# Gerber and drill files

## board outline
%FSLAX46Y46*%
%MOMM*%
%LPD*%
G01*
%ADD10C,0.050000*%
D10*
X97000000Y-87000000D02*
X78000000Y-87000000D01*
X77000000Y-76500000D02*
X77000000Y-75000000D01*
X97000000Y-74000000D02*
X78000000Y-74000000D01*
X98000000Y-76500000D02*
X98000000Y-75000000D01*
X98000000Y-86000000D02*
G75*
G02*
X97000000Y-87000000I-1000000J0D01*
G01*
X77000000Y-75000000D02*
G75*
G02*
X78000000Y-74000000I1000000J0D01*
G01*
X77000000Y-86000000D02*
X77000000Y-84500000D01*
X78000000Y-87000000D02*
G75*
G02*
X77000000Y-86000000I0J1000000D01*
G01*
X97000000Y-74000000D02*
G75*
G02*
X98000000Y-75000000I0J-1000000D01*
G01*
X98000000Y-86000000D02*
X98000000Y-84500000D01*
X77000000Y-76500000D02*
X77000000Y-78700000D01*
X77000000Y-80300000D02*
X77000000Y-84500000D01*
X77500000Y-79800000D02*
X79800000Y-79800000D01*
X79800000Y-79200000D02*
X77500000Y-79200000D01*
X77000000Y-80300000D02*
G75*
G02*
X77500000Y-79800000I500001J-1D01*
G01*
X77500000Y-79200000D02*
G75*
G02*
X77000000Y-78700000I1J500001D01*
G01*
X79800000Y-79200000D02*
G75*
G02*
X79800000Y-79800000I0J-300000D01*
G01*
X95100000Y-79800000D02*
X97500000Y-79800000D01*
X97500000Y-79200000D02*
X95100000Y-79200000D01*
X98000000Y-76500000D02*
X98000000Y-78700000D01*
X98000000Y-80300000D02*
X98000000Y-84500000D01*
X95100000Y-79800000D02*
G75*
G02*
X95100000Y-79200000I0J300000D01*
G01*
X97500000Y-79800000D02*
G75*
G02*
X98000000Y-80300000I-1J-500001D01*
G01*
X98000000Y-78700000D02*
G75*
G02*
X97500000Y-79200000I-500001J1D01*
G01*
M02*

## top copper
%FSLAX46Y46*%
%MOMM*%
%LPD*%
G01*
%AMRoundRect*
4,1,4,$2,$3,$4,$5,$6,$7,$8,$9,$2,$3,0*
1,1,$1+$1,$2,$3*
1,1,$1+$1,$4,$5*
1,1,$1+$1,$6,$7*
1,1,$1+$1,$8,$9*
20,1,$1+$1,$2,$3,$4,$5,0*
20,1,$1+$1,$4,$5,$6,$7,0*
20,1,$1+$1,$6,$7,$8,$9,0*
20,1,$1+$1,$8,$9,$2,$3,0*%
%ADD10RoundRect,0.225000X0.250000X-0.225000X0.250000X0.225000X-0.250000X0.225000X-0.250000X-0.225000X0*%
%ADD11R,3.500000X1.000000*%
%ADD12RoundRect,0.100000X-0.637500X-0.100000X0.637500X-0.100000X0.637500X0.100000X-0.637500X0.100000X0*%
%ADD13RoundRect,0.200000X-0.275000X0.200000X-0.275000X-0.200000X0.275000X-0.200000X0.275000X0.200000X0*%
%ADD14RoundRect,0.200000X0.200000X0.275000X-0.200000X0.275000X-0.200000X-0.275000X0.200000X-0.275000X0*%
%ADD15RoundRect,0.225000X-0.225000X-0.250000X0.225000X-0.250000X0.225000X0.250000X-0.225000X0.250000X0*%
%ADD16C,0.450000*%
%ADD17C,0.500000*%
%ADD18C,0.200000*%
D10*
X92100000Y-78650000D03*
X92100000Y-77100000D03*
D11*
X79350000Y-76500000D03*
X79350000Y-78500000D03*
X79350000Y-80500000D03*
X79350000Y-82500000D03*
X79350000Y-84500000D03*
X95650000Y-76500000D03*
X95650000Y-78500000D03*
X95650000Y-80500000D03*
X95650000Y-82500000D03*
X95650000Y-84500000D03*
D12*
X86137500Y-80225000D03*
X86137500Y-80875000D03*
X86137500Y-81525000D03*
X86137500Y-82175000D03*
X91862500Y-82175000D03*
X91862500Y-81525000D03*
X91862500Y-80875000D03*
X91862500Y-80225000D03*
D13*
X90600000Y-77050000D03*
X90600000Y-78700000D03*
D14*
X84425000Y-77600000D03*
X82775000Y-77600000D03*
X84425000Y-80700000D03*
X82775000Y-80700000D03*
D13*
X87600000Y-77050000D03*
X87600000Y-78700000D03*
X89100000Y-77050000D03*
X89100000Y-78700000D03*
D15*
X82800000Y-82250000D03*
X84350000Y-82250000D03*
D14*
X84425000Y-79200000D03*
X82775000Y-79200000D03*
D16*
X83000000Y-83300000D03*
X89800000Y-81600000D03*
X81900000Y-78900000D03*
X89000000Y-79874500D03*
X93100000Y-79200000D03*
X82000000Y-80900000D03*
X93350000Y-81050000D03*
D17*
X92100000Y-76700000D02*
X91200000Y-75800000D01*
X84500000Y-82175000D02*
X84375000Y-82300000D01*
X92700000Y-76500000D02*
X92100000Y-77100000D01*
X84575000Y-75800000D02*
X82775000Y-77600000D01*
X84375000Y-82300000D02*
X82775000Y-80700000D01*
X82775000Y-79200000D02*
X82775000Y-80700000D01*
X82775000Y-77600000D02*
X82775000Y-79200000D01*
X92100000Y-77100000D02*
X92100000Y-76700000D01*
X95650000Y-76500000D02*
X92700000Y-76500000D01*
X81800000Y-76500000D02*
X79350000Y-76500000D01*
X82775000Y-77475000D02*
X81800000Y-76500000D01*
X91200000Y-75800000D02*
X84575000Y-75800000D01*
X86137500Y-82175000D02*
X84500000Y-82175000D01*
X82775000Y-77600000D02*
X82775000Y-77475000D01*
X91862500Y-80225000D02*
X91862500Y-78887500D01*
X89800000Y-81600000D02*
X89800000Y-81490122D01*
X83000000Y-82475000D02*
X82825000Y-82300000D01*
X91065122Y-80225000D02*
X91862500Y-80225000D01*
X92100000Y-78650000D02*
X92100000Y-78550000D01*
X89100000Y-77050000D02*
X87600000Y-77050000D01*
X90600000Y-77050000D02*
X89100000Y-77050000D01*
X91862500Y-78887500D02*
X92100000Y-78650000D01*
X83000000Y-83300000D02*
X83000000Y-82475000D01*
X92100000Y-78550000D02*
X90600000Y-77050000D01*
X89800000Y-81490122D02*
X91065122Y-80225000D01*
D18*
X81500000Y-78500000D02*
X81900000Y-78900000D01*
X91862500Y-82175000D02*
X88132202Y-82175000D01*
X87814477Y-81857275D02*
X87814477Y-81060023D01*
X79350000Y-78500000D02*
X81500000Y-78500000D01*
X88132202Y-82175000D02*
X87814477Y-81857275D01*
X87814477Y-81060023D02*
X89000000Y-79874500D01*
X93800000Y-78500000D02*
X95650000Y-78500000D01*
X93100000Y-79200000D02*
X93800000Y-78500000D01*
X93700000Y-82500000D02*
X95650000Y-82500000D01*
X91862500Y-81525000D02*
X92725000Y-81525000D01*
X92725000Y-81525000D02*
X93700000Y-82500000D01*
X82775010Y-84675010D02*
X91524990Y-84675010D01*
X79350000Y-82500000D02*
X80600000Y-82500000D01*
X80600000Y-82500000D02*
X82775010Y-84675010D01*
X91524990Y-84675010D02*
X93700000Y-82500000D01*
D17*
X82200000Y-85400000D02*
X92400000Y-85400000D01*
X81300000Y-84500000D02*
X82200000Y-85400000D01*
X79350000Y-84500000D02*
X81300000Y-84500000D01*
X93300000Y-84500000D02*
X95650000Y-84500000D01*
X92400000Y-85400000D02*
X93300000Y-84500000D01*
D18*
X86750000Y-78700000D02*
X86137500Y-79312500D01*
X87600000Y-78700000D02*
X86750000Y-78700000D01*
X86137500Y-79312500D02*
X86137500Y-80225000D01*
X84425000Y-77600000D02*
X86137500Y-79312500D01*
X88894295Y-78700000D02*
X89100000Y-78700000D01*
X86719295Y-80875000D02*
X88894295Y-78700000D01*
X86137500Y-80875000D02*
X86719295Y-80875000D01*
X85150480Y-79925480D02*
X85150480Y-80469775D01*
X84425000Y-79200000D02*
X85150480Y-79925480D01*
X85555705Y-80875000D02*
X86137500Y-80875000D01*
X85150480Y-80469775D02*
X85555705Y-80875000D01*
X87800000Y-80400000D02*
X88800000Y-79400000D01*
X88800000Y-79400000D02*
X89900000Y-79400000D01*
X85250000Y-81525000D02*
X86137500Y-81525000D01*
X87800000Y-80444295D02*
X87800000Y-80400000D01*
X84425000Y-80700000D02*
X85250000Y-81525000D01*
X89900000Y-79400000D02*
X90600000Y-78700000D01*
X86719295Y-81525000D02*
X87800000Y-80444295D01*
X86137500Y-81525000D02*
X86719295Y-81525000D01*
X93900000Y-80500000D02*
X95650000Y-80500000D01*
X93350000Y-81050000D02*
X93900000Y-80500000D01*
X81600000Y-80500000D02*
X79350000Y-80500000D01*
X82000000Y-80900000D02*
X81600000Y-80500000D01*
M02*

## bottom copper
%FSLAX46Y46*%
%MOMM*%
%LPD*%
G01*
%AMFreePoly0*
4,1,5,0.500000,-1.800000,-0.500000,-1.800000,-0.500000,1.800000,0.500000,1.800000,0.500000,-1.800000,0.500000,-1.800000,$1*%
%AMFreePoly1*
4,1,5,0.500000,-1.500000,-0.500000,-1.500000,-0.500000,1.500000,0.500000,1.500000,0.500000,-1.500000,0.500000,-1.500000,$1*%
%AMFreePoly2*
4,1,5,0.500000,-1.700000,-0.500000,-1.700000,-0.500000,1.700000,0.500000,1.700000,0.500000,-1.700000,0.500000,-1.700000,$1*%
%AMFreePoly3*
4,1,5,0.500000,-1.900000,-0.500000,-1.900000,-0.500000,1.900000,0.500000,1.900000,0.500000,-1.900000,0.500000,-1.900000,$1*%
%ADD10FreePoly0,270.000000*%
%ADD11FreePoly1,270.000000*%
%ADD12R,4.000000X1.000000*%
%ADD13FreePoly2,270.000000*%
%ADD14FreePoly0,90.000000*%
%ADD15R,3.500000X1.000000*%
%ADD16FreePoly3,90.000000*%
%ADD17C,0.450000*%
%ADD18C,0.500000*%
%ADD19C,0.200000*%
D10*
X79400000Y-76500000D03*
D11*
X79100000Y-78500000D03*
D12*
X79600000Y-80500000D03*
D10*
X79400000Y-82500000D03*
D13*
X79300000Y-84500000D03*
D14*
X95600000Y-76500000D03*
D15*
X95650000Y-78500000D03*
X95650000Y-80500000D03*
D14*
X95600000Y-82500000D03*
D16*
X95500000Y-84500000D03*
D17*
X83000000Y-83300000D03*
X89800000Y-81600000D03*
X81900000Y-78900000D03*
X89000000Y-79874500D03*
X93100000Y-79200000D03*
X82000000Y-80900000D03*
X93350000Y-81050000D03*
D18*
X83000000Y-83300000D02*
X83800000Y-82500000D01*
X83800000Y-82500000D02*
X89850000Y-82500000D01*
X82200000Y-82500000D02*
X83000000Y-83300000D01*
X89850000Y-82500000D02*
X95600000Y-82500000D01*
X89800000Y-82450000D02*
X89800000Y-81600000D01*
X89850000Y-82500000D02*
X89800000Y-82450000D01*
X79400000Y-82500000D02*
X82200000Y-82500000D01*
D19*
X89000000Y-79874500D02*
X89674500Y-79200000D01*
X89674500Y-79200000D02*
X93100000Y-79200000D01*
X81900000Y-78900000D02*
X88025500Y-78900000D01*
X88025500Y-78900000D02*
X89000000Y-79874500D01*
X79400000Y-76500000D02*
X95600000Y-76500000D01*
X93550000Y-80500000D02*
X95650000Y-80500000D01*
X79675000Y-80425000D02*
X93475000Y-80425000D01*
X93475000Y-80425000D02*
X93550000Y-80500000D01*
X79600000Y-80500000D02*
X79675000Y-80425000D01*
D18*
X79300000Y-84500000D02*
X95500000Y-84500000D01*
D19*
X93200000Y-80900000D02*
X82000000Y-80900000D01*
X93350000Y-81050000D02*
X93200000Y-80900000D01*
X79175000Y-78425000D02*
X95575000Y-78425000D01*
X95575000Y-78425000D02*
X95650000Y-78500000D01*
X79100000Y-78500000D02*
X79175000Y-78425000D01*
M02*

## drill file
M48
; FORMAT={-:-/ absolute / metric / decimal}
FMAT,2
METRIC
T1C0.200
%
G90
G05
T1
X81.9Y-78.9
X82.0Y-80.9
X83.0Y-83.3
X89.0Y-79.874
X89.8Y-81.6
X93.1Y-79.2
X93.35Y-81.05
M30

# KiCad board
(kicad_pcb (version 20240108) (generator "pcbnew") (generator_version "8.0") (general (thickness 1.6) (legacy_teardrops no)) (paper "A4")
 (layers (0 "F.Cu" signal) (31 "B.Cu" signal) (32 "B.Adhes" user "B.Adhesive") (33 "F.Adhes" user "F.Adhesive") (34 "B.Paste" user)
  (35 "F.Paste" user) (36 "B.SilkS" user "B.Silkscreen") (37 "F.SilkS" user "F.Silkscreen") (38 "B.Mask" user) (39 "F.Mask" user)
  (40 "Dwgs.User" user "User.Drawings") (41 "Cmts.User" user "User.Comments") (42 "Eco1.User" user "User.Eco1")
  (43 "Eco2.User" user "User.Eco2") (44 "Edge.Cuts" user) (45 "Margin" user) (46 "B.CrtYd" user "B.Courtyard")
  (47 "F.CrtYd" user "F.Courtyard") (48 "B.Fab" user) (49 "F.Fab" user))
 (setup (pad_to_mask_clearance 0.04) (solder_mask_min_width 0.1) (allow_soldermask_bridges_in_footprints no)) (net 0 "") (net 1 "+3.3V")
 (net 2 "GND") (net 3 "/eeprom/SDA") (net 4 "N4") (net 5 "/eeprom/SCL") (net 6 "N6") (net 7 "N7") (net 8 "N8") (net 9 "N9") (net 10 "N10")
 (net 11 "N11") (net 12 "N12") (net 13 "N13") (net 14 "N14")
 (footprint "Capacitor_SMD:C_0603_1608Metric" (layer "F.Cu") (at 92.1 77.875 90)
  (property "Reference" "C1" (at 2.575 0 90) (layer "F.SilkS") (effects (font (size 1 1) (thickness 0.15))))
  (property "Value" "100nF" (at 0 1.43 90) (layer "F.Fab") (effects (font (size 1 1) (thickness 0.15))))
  (pad "1" smd roundrect (at -0.775 0 90) (size 0.9 0.95) (layers "F.Cu" "F.Paste" "F.Mask") (roundrect_rratio 0.25) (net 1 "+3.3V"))
  (pad "2" smd roundrect (at 0.775 0 90) (size 0.9 0.95) (layers "F.Cu" "F.Paste" "F.Mask") (roundrect_rratio 0.25) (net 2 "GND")))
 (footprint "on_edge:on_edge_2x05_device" (layer "F.Cu") (at 77 80.5 -90)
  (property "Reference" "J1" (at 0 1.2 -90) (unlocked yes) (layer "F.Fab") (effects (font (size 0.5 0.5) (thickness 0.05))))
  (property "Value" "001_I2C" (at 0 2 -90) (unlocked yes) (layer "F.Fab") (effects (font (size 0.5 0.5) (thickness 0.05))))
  (fp_line (start -4 0) (end -1.8 0) (stroke (width 0.05) (type solid)) (layer "Edge.Cuts"))
  (fp_line (start -0.2 0) (end 4 0) (stroke (width 0.05) (type solid)) (layer "Edge.Cuts"))
  (fp_line (start -0.7 -0.5) (end -0.7 -2.8) (stroke (width 0.05) (type solid)) (layer "Edge.Cuts"))
  (fp_line (start -1.3 -2.8) (end -1.3 -0.5) (stroke (width 0.05) (type solid)) (layer "Edge.Cuts"))
  (fp_arc (start -0.2 0) (mid -0.553553 -0.146447) (end -0.7 -0.5) (stroke (width 0.05) (type solid)) (layer "Edge.Cuts"))
  (fp_arc (start -1.3 -0.5) (mid -1.446447 -0.146447) (end -1.8 0) (stroke (width 0.05) (type solid)) (layer "Edge.Cuts"))
  (fp_arc (start -1.3 -2.8) (mid -1 -3.1) (end -0.7 -2.8) (stroke (width 0.05) (type solid)) (layer "Edge.Cuts"))
  (pad "1" smd rect (at -4 -2.35 90) (size 1 3.5) (layers "F.Cu" "F.Mask") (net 2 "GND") (zone_connect 0))
  (pad "2" smd rect (at -2 -2.35 270) (size 1 3.5) (layers "F.Cu" "F.Mask") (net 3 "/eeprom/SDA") (zone_connect 0))
  (pad "3" smd rect (at 0 -2.35 270) (size 1 3.5) (layers "F.Cu" "F.Mask") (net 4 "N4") (zone_connect 0))
  (pad "4" smd rect (at 2 -2.35 90) (size 1 3.5) (layers "F.Cu" "F.Mask") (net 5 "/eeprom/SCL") (zone_connect 0))
  (pad "5" smd rect (at 4 -2.35 90) (size 1 3.5) (layers "F.Cu" "F.Mask") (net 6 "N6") (zone_connect 0))
  (pad "6" smd custom (at -4 -2.4 270) (size 1 3.6) (layers "B.Cu" "B.Mask") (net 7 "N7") (zone_connect 0)
   (options (clearance outline) (anchor rect)) (primitives))
  (pad "7" smd custom (at -2 -2.1 270) (size 1 3) (layers "B.Cu" "B.Mask") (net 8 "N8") (zone_connect 0)
   (options (clearance outline) (anchor rect)) (primitives))
  (pad "8" smd rect (at 0 -2.6 270) (size 1 4) (layers "B.Cu" "B.Mask") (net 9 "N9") (zone_connect 0))
  (pad "9" smd custom (at 2 -2.4 270) (size 1 3.6) (layers "B.Cu" "B.Mask") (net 1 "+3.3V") (zone_connect 0)
   (options (clearance outline) (anchor rect)) (primitives))
  (pad "10" smd custom (at 4 -2.3 270) (size 1 3.4) (layers "B.Cu" "B.Mask") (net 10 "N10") (zone_connect 0)
   (options (clearance outline) (anchor rect)) (primitives))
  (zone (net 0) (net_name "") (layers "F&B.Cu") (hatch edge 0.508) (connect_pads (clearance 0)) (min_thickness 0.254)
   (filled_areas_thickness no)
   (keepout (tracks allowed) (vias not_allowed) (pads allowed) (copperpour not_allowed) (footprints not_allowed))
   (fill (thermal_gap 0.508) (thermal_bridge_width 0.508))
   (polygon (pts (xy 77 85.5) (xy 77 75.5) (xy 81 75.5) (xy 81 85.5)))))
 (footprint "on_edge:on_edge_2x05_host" (layer "F.Cu") (at 98 80.5 -90)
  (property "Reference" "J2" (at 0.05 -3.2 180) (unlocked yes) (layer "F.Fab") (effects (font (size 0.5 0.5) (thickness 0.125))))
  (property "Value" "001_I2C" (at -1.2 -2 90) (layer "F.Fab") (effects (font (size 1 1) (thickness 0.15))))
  (fp_line (start -0.7 2.9) (end -0.7 0.5) (stroke (width 0.05) (type solid)) (layer "Edge.Cuts"))
  (fp_line (start -1.3 0.5) (end -1.3 2.9) (stroke (width 0.05) (type solid)) (layer "Edge.Cuts"))
  (fp_line (start -4 0) (end -1.8 0) (stroke (width 0.05) (type solid)) (layer "Edge.Cuts"))
  (fp_line (start -0.2 0) (end 4 0) (stroke (width 0.05) (type solid)) (layer "Edge.Cuts"))
  (fp_arc (start -0.7 2.9) (mid -1 3.2) (end -1.3 2.9) (stroke (width 0.05) (type solid)) (layer "Edge.Cuts"))
  (fp_arc (start -0.7 0.5) (mid -0.553553 0.146447) (end -0.2 0) (stroke (width 0.05) (type solid)) (layer "Edge.Cuts"))
  (fp_arc (start -1.8 0) (mid -1.446447 0.146447) (end -1.3 0.5) (stroke (width 0.05) (type solid)) (layer "Edge.Cuts"))
  (pad "1" smd rect (at -4 2.35 270) (size 1 3.5) (layers "F.Cu" "F.Mask") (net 2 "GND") (zone_connect 0))
  (pad "2" smd rect (at -2 2.35 270) (size 1 3.5) (layers "F.Cu" "F.Mask") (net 3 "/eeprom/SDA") (zone_connect 0))
  (pad "3" smd rect (at 0 2.35 270) (size 1 3.5) (layers "F.Cu" "F.Mask") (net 4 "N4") (zone_connect 0))
  (pad "4" smd rect (at 2 2.35 270) (size 1 3.5) (layers "F.Cu" "F.Mask") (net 5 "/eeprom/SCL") (zone_connect 0))
  (pad "5" smd rect (at 4 2.35 270) (size 1 3.5) (layers "F.Cu" "F.Mask") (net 6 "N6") (zone_connect 0))
  (pad "6" smd custom (at -4 2.4 90) (size 1 3.6) (layers "B.Cu" "B.Mask") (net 7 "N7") (zone_connect 0)
   (options (clearance outline) (anchor rect)) (primitives))
  (pad "7" smd rect (at -2 2.35 90) (size 1 3.5) (layers "B.Cu" "B.Mask") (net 8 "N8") (zone_connect 0))
  (pad "8" smd rect (at 0 2.35 90) (size 1 3.5) (layers "B.Cu" "B.Mask") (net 9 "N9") (zone_connect 0))
  (pad "9" smd custom (at 2 2.4 90) (size 1 3.6) (layers "B.Cu" "B.Mask") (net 1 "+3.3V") (zone_connect 0)
   (options (clearance outline) (anchor rect)) (primitives))
  (pad "10" smd custom (at 4 2.5 90) (size 1 3.8) (layers "B.Cu" "B.Mask") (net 10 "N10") (zone_connect 0)
   (options (clearance outline) (anchor rect)) (primitives))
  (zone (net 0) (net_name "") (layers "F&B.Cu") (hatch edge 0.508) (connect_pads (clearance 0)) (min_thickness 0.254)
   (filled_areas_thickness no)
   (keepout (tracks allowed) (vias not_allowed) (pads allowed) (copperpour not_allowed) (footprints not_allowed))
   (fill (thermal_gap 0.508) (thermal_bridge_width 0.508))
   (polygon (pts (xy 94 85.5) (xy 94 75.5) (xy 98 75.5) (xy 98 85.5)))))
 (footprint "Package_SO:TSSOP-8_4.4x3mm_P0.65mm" (layer "F.Cu") (at 89 81.2)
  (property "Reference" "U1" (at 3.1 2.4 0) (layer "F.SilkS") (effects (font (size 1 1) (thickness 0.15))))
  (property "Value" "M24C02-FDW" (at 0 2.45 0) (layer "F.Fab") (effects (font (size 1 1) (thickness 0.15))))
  (pad "1" smd roundrect (at -2.8625 -0.975) (size 1.475 0.4) (layers "F.Cu" "F.Paste" "F.Mask") (roundrect_rratio 0.25) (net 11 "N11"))
  (pad "2" smd roundrect (at -2.8625 -0.325) (size 1.475 0.4) (layers "F.Cu" "F.Paste" "F.Mask") (roundrect_rratio 0.25) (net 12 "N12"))
  (pad "3" smd roundrect (at -2.8625 0.325) (size 1.475 0.4) (layers "F.Cu" "F.Paste" "F.Mask") (roundrect_rratio 0.25) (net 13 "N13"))
  (pad "4" smd roundrect (at -2.8625 0.975) (size 1.475 0.4) (layers "F.Cu" "F.Paste" "F.Mask") (roundrect_rratio 0.25) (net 2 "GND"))
  (pad "5" smd roundrect (at 2.8625 0.975) (size 1.475 0.4) (layers "F.Cu" "F.Paste" "F.Mask") (roundrect_rratio 0.25) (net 3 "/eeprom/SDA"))
  (pad "6" smd roundrect (at 2.8625 0.325) (size 1.475 0.4) (layers "F.Cu" "F.Paste" "F.Mask") (roundrect_rratio 0.25) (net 5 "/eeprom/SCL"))
  (pad "7" smd roundrect (at 2.8625 -0.325) (size 1.475 0.4) (layers "F.Cu" "F.Paste" "F.Mask") (roundrect_rratio 0.25) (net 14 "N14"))
  (pad "8" smd roundrect (at 2.8625 -0.975) (size 1.475 0.4) (layers "F.Cu" "F.Paste" "F.Mask") (roundrect_rratio 0.25) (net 1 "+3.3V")))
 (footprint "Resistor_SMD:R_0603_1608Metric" (layer "F.Cu") (at 90.6 77.875 -90)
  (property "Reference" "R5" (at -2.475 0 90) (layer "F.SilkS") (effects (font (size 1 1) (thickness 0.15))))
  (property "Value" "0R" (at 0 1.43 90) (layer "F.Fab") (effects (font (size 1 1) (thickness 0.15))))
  (pad "1" smd roundrect (at -0.825 0 270) (size 0.8 0.95) (layers "F.Cu" "F.Paste" "F.Mask") (roundrect_rratio 0.25) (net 1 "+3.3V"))
  (pad "2" smd roundrect (at 0.825 0 270) (size 0.8 0.95) (layers "F.Cu" "F.Paste" "F.Mask") (roundrect_rratio 0.25) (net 13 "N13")))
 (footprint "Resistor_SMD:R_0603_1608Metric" (layer "F.Cu") (at 83.6 77.6 180)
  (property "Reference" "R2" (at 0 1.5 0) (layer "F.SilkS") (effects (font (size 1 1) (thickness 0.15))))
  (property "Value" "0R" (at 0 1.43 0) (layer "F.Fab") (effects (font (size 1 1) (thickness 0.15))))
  (pad "1" smd roundrect (at -0.825 0 180) (size 0.8 0.95) (layers "F.Cu" "F.Paste" "F.Mask") (roundrect_rratio 0.25) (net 11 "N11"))
  (pad "2" smd roundrect (at 0.825 0 180) (size 0.8 0.95) (layers "F.Cu" "F.Paste" "F.Mask") (roundrect_rratio 0.25) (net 2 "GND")))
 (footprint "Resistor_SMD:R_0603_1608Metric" (layer "F.Cu") (at 83.6 80.7 180)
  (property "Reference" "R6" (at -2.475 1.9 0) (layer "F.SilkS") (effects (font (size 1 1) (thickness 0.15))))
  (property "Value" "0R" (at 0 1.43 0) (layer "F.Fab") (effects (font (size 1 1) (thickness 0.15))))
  (pad "1" smd roundrect (at -0.825 0 180) (size 0.8 0.95) (layers "F.Cu" "F.Paste" "F.Mask") (roundrect_rratio 0.25) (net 13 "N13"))
  (pad "2" smd roundrect (at 0.825 0 180) (size 0.8 0.95) (layers "F.Cu" "F.Paste" "F.Mask") (roundrect_rratio 0.25) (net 2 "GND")))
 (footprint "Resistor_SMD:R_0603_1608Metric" (layer "F.Cu") (at 87.6 77.875 -90)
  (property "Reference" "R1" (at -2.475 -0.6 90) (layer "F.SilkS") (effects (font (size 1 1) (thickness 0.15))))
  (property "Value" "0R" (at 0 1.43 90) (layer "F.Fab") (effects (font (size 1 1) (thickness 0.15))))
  (pad "1" smd roundrect (at -0.825 0 270) (size 0.8 0.95) (layers "F.Cu" "F.Paste" "F.Mask") (roundrect_rratio 0.25) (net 1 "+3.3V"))
  (pad "2" smd roundrect (at 0.825 0 270) (size 0.8 0.95) (layers "F.Cu" "F.Paste" "F.Mask") (roundrect_rratio 0.25) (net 11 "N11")))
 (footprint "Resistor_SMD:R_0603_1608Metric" (layer "F.Cu") (at 89.1 77.875 -90)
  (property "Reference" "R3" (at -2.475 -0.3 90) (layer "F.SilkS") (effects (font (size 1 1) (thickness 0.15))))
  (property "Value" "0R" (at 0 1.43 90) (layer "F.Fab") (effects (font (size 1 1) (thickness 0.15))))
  (pad "1" smd roundrect (at -0.825 0 270) (size 0.8 0.95) (layers "F.Cu" "F.Paste" "F.Mask") (roundrect_rratio 0.25) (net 1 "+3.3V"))
  (pad "2" smd roundrect (at 0.825 0 270) (size 0.8 0.95) (layers "F.Cu" "F.Paste" "F.Mask") (roundrect_rratio 0.25) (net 12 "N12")))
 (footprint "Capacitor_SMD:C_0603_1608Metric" (layer "F.Cu") (at 83.575 82.25)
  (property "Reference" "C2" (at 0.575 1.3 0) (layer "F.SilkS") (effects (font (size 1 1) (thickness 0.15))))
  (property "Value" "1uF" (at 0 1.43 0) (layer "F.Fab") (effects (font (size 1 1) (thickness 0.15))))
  (pad "1" smd roundrect (at -0.775 0) (size 0.9 0.95) (layers "F.Cu" "F.Paste" "F.Mask") (roundrect_rratio 0.25) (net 1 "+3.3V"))
  (pad "2" smd roundrect (at 0.775 0) (size 0.9 0.95) (layers "F.Cu" "F.Paste" "F.Mask") (roundrect_rratio 0.25) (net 2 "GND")))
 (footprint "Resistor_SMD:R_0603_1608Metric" (layer "F.Cu") (at 83.6 79.2 180)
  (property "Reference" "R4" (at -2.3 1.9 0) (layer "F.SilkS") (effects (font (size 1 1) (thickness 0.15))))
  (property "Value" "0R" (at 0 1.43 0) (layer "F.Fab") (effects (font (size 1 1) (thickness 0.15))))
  (pad "1" smd roundrect (at -0.825 0 180) (size 0.8 0.95) (layers "F.Cu" "F.Paste" "F.Mask") (roundrect_rratio 0.25) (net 12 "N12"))
  (pad "2" smd roundrect (at 0.825 0 180) (size 0.8 0.95) (layers "F.Cu" "F.Paste" "F.Mask") (roundrect_rratio 0.25) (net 2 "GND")))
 (gr_line (start 97 87) (end 78 87) (stroke (width 0.05) (type solid)) (layer "Edge.Cuts"))
 (gr_line (start 77 76.5) (end 77 75) (stroke (width 0.05) (type solid)) (layer "Edge.Cuts"))
 (gr_line (start 97 74) (end 78 74) (stroke (width 0.05) (type solid)) (layer "Edge.Cuts"))
 (gr_line (start 98 76.5) (end 98 75) (stroke (width 0.05) (type solid)) (layer "Edge.Cuts"))
 (gr_arc (start 98 86) (mid 97.707107 86.707107) (end 97 87) (stroke (width 0.05) (type solid)) (layer "Edge.Cuts"))
 (gr_arc (start 77 75) (mid 77.292893 74.292893) (end 78 74) (stroke (width 0.05) (type solid)) (layer "Edge.Cuts"))
 (gr_line (start 77 86) (end 77 84.5) (stroke (width 0.05) (type solid)) (layer "Edge.Cuts"))
 (gr_arc (start 78 87) (mid 77.292893 86.707107) (end 77 86) (stroke (width 0.05) (type solid)) (layer "Edge.Cuts"))
 (gr_arc (start 97 74) (mid 97.707107 74.292893) (end 98 75) (stroke (width 0.05) (type solid)) (layer "Edge.Cuts"))
 (gr_line (start 98 86) (end 98 84.5) (stroke (width 0.05) (type solid)) (layer "Edge.Cuts"))
 (segment (start 92.1 76.7) (end 91.2 75.8) (width 0.5) (layer "F.Cu") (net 2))
 (segment (start 84.5 82.175) (end 84.375 82.3) (width 0.5) (layer "F.Cu") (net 2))
 (segment (start 92.7 76.5) (end 92.1 77.1) (width 0.5) (layer "F.Cu") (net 2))
 (segment (start 84.575 75.8) (end 82.775 77.6) (width 0.5) (layer "F.Cu") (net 2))
 (segment (start 84.375 82.3) (end 82.775 80.7) (width 0.5) (layer "F.Cu") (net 2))
 (segment (start 82.775 79.2) (end 82.775 80.7) (width 0.5) (layer "F.Cu") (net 2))
 (segment (start 82.775 77.6) (end 82.775 79.2) (width 0.5) (layer "F.Cu") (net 2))
 (segment (start 92.1 77.1) (end 92.1 76.7) (width 0.5) (layer "F.Cu") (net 2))
 (segment (start 95.65 76.5) (end 92.7 76.5) (width 0.5) (layer "F.Cu") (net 2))
 (segment (start 81.8 76.5) (end 79.35 76.5) (width 0.5) (layer "F.Cu") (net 2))
 (segment (start 82.775 77.475) (end 81.8 76.5) (width 0.5) (layer "F.Cu") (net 2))
 (segment (start 91.2 75.8) (end 84.575 75.8) (width 0.5) (layer "F.Cu") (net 2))
 (segment (start 86.1375 82.175) (end 84.5 82.175) (width 0.5) (layer "F.Cu") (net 2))
 (segment (start 82.775 77.6) (end 82.775 77.475) (width 0.5) (layer "F.Cu") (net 2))
 (segment (start 91.8625 80.225) (end 91.8625 78.8875) (width 0.5) (layer "F.Cu") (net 1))
 (segment (start 89.8 81.6) (end 89.8 81.490122) (width 0.5) (layer "F.Cu") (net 1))
 (segment (start 83 82.475) (end 82.825 82.3) (width 0.5) (layer "F.Cu") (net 1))
 (segment (start 91.065122 80.225) (end 91.8625 80.225) (width 0.5) (layer "F.Cu") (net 1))
 (segment (start 92.1 78.65) (end 92.1 78.55) (width 0.5) (layer "F.Cu") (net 1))
 (segment (start 89.1 77.05) (end 87.6 77.05) (width 0.5) (layer "F.Cu") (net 1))
 (segment (start 90.6 77.05) (end 89.1 77.05) (width 0.5) (layer "F.Cu") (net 1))
 (segment (start 91.8625 78.8875) (end 92.1 78.65) (width 0.5) (layer "F.Cu") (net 1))
 (segment (start 83 83.3) (end 83 82.475) (width 0.5) (layer "F.Cu") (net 1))
 (segment (start 92.1 78.55) (end 90.6 77.05) (width 0.5) (layer "F.Cu") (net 1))
 (segment (start 89.8 81.490122) (end 91.065122 80.225) (width 0.5) (layer "F.Cu") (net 1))
 (via (at 83 83.3) (size 0.45) (drill 0.2) (layers "F.Cu" "B.Cu") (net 1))
 (via (at 89.8 81.6) (size 0.45) (drill 0.2) (layers "F.Cu" "B.Cu") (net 1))
 (segment (start 83 83.3) (end 83.8 82.5) (width 0.5) (layer "B.Cu") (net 1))
 (segment (start 83.8 82.5) (end 89.85 82.5) (width 0.5) (layer "B.Cu") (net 1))
 (segment (start 82.2 82.5) (end 83 83.3) (width 0.5) (layer "B.Cu") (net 1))
 (segment (start 89.85 82.5) (end 95.6 82.5) (width 0.5) (layer "B.Cu") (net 1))
 (segment (start 89.8 82.45) (end 89.8 81.6) (width 0.5) (layer "B.Cu") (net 1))
 (segment (start 89.85 82.5) (end 89.8 82.45) (width 0.5) (layer "B.Cu") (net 1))
 (segment (start 79.4 82.5) (end 82.2 82.5) (width 0.5) (layer "B.Cu") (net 1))
 (segment (start 81.5 78.5) (end 81.9 78.9) (width 0.2) (layer "F.Cu") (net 3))
 (segment (start 91.8625 82.175) (end 88.132202 82.175) (width 0.2) (layer "F.Cu") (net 3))
 (segment (start 87.814477 81.857275) (end 87.814477 81.060023) (width 0.2) (layer "F.Cu") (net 3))
 (segment (start 79.35 78.5) (end 81.5 78.5) (width 0.2) (layer "F.Cu") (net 3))
 (segment (start 88.132202 82.175) (end 87.814477 81.857275) (width 0.2) (layer "F.Cu") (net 3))
 (segment (start 87.814477 81.060023) (end 89 79.8745) (width 0.2) (layer "F.Cu") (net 3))
 (segment (start 93.8 78.5) (end 95.65 78.5) (width 0.2) (layer "F.Cu") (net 3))
 (segment (start 93.1 79.2) (end 93.8 78.5) (width 0.2) (layer "F.Cu") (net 3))
 (via (at 81.9 78.9) (size 0.45) (drill 0.2) (layers "F.Cu" "B.Cu") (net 3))
 (via (at 89 79.8745) (size 0.45) (drill 0.2) (layers "F.Cu" "B.Cu") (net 3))
 (via (at 93.1 79.2) (size 0.45) (drill 0.2) (layers "F.Cu" "B.Cu") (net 3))
 (segment (start 89 79.8745) (end 89.6745 79.2) (width 0.2) (layer "B.Cu") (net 3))
 (segment (start 89.6745 79.2) (end 93.1 79.2) (width 0.2) (layer "B.Cu") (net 3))
 (segment (start 81.9 78.9) (end 88.0255 78.9) (width 0.2) (layer "B.Cu") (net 3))
 (segment (start 88.0255 78.9) (end 89 79.8745) (width 0.2) (layer "B.Cu") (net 3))
 (segment (start 93.7 82.5) (end 95.65 82.5) (width 0.2) (layer "F.Cu") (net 5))
 (segment (start 91.8625 81.525) (end 92.725 81.525) (width 0.2) (layer "F.Cu") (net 5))
 (segment (start 92.725 81.525) (end 93.7 82.5) (width 0.2) (layer "F.Cu") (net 5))
 (segment (start 82.77501 84.67501) (end 91.52499 84.67501) (width 0.2) (layer "F.Cu") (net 5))
 (segment (start 79.35 82.5) (end 80.6 82.5) (width 0.2) (layer "F.Cu") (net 5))
 (segment (start 80.6 82.5) (end 82.77501 84.67501) (width 0.2) (layer "F.Cu") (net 5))
 (segment (start 91.52499 84.67501) (end 93.7 82.5) (width 0.2) (layer "F.Cu") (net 5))
 (segment (start 79.4 76.5) (end 95.6 76.5) (width 0.2) (layer "B.Cu") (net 7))
 (segment (start 82.2 85.4) (end 92.4 85.4) (width 0.5) (layer "F.Cu") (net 6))
 (segment (start 81.3 84.5) (end 82.2 85.4) (width 0.5) (layer "F.Cu") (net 6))
 (segment (start 79.35 84.5) (end 81.3 84.5) (width 0.5) (layer "F.Cu") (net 6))
 (segment (start 93.3 84.5) (end 95.65 84.5) (width 0.5) (layer "F.Cu") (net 6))
 (segment (start 92.4 85.4) (end 93.3 84.5) (width 0.5) (layer "F.Cu") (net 6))
 (segment (start 93.55 80.5) (end 95.65 80.5) (width 0.2) (layer "B.Cu") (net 9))
 (segment (start 79.675 80.425) (end 93.475 80.425) (width 0.2) (layer "B.Cu") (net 9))
 (segment (start 93.475 80.425) (end 93.55 80.5) (width 0.2) (layer "B.Cu") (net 9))
 (segment (start 79.6 80.5) (end 79.675 80.425) (width 0.2) (layer "B.Cu") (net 9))
 (segment (start 79.3 84.5) (end 95.5 84.5) (width 0.5) (layer "B.Cu") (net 10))
 (segment (start 86.75 78.7) (end 86.1375 79.3125) (width 0.2) (layer "F.Cu") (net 11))
 (segment (start 87.6 78.7) (end 86.75 78.7) (width 0.2) (layer "F.Cu") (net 11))
 (segment (start 86.1375 79.3125) (end 86.1375 80.225) (width 0.2) (layer "F.Cu") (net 11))
 (segment (start 84.425 77.6) (end 86.1375 79.3125) (width 0.2) (layer "F.Cu") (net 11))
 (segment (start 88.894295 78.7) (end 89.1 78.7) (width 0.2) (layer "F.Cu") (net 12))
 (segment (start 86.719295 80.875) (end 88.894295 78.7) (width 0.2) (layer "F.Cu") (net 12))
 (segment (start 86.1375 80.875) (end 86.719295 80.875) (width 0.2) (layer "F.Cu") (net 12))
 (segment (start 85.15048 79.92548) (end 85.15048 80.469775) (width 0.2) (layer "F.Cu") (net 12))
 (segment (start 84.425 79.2) (end 85.15048 79.92548) (width 0.2) (layer "F.Cu") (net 12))
 (segment (start 85.555705 80.875) (end 86.1375 80.875) (width 0.2) (layer "F.Cu") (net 12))
 (segment (start 85.15048 80.469775) (end 85.555705 80.875) (width 0.2) (layer "F.Cu") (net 12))
 (segment (start 87.8 80.4) (end 88.8 79.4) (width 0.2) (layer "F.Cu") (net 13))
 (segment (start 88.8 79.4) (end 89.9 79.4) (width 0.2) (layer "F.Cu") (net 13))
 (segment (start 85.25 81.525) (end 86.1375 81.525) (width 0.2) (layer "F.Cu") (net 13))
 (segment (start 87.8 80.444295) (end 87.8 80.4) (width 0.2) (layer "F.Cu") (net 13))
 (segment (start 84.425 80.7) (end 85.25 81.525) (width 0.2) (layer "F.Cu") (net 13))
 (segment (start 89.9 79.4) (end 90.6 78.7) (width 0.2) (layer "F.Cu") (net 13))
 (segment (start 86.719295 81.525) (end 87.8 80.444295) (width 0.2) (layer "F.Cu") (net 13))
 (segment (start 86.1375 81.525) (end 86.719295 81.525) (width 0.2) (layer "F.Cu") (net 13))
 (segment (start 93.9 80.5) (end 95.65 80.5) (width 0.2) (layer "F.Cu") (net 4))
 (segment (start 93.35 81.05) (end 93.9 80.5) (width 0.2) (layer "F.Cu") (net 4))
 (segment (start 81.6 80.5) (end 79.35 80.5) (width 0.2) (layer "F.Cu") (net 4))
 (segment (start 82 80.9) (end 81.6 80.5) (width 0.2) (layer "F.Cu") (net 4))
 (via (at 82 80.9) (size 0.45) (drill 0.2) (layers "F.Cu" "B.Cu") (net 4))
 (via (at 93.35 81.05) (size 0.45) (drill 0.2) (layers "F.Cu" "B.Cu") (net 4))
 (segment (start 93.2 80.9) (end 82 80.9) (width 0.2) (layer "B.Cu") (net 4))
 (segment (start 93.35 81.05) (end 93.2 80.9) (width 0.2) (layer "B.Cu") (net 4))
 (segment (start 79.175 78.425) (end 95.575 78.425) (width 0.2) (layer "B.Cu") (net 8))
 (segment (start 95.575 78.425) (end 95.65 78.5) (width 0.2) (layer "B.Cu") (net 8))
 (segment (start 79.1 78.5) (end 79.175 78.425) (width 0.2) (layer "B.Cu") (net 8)))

